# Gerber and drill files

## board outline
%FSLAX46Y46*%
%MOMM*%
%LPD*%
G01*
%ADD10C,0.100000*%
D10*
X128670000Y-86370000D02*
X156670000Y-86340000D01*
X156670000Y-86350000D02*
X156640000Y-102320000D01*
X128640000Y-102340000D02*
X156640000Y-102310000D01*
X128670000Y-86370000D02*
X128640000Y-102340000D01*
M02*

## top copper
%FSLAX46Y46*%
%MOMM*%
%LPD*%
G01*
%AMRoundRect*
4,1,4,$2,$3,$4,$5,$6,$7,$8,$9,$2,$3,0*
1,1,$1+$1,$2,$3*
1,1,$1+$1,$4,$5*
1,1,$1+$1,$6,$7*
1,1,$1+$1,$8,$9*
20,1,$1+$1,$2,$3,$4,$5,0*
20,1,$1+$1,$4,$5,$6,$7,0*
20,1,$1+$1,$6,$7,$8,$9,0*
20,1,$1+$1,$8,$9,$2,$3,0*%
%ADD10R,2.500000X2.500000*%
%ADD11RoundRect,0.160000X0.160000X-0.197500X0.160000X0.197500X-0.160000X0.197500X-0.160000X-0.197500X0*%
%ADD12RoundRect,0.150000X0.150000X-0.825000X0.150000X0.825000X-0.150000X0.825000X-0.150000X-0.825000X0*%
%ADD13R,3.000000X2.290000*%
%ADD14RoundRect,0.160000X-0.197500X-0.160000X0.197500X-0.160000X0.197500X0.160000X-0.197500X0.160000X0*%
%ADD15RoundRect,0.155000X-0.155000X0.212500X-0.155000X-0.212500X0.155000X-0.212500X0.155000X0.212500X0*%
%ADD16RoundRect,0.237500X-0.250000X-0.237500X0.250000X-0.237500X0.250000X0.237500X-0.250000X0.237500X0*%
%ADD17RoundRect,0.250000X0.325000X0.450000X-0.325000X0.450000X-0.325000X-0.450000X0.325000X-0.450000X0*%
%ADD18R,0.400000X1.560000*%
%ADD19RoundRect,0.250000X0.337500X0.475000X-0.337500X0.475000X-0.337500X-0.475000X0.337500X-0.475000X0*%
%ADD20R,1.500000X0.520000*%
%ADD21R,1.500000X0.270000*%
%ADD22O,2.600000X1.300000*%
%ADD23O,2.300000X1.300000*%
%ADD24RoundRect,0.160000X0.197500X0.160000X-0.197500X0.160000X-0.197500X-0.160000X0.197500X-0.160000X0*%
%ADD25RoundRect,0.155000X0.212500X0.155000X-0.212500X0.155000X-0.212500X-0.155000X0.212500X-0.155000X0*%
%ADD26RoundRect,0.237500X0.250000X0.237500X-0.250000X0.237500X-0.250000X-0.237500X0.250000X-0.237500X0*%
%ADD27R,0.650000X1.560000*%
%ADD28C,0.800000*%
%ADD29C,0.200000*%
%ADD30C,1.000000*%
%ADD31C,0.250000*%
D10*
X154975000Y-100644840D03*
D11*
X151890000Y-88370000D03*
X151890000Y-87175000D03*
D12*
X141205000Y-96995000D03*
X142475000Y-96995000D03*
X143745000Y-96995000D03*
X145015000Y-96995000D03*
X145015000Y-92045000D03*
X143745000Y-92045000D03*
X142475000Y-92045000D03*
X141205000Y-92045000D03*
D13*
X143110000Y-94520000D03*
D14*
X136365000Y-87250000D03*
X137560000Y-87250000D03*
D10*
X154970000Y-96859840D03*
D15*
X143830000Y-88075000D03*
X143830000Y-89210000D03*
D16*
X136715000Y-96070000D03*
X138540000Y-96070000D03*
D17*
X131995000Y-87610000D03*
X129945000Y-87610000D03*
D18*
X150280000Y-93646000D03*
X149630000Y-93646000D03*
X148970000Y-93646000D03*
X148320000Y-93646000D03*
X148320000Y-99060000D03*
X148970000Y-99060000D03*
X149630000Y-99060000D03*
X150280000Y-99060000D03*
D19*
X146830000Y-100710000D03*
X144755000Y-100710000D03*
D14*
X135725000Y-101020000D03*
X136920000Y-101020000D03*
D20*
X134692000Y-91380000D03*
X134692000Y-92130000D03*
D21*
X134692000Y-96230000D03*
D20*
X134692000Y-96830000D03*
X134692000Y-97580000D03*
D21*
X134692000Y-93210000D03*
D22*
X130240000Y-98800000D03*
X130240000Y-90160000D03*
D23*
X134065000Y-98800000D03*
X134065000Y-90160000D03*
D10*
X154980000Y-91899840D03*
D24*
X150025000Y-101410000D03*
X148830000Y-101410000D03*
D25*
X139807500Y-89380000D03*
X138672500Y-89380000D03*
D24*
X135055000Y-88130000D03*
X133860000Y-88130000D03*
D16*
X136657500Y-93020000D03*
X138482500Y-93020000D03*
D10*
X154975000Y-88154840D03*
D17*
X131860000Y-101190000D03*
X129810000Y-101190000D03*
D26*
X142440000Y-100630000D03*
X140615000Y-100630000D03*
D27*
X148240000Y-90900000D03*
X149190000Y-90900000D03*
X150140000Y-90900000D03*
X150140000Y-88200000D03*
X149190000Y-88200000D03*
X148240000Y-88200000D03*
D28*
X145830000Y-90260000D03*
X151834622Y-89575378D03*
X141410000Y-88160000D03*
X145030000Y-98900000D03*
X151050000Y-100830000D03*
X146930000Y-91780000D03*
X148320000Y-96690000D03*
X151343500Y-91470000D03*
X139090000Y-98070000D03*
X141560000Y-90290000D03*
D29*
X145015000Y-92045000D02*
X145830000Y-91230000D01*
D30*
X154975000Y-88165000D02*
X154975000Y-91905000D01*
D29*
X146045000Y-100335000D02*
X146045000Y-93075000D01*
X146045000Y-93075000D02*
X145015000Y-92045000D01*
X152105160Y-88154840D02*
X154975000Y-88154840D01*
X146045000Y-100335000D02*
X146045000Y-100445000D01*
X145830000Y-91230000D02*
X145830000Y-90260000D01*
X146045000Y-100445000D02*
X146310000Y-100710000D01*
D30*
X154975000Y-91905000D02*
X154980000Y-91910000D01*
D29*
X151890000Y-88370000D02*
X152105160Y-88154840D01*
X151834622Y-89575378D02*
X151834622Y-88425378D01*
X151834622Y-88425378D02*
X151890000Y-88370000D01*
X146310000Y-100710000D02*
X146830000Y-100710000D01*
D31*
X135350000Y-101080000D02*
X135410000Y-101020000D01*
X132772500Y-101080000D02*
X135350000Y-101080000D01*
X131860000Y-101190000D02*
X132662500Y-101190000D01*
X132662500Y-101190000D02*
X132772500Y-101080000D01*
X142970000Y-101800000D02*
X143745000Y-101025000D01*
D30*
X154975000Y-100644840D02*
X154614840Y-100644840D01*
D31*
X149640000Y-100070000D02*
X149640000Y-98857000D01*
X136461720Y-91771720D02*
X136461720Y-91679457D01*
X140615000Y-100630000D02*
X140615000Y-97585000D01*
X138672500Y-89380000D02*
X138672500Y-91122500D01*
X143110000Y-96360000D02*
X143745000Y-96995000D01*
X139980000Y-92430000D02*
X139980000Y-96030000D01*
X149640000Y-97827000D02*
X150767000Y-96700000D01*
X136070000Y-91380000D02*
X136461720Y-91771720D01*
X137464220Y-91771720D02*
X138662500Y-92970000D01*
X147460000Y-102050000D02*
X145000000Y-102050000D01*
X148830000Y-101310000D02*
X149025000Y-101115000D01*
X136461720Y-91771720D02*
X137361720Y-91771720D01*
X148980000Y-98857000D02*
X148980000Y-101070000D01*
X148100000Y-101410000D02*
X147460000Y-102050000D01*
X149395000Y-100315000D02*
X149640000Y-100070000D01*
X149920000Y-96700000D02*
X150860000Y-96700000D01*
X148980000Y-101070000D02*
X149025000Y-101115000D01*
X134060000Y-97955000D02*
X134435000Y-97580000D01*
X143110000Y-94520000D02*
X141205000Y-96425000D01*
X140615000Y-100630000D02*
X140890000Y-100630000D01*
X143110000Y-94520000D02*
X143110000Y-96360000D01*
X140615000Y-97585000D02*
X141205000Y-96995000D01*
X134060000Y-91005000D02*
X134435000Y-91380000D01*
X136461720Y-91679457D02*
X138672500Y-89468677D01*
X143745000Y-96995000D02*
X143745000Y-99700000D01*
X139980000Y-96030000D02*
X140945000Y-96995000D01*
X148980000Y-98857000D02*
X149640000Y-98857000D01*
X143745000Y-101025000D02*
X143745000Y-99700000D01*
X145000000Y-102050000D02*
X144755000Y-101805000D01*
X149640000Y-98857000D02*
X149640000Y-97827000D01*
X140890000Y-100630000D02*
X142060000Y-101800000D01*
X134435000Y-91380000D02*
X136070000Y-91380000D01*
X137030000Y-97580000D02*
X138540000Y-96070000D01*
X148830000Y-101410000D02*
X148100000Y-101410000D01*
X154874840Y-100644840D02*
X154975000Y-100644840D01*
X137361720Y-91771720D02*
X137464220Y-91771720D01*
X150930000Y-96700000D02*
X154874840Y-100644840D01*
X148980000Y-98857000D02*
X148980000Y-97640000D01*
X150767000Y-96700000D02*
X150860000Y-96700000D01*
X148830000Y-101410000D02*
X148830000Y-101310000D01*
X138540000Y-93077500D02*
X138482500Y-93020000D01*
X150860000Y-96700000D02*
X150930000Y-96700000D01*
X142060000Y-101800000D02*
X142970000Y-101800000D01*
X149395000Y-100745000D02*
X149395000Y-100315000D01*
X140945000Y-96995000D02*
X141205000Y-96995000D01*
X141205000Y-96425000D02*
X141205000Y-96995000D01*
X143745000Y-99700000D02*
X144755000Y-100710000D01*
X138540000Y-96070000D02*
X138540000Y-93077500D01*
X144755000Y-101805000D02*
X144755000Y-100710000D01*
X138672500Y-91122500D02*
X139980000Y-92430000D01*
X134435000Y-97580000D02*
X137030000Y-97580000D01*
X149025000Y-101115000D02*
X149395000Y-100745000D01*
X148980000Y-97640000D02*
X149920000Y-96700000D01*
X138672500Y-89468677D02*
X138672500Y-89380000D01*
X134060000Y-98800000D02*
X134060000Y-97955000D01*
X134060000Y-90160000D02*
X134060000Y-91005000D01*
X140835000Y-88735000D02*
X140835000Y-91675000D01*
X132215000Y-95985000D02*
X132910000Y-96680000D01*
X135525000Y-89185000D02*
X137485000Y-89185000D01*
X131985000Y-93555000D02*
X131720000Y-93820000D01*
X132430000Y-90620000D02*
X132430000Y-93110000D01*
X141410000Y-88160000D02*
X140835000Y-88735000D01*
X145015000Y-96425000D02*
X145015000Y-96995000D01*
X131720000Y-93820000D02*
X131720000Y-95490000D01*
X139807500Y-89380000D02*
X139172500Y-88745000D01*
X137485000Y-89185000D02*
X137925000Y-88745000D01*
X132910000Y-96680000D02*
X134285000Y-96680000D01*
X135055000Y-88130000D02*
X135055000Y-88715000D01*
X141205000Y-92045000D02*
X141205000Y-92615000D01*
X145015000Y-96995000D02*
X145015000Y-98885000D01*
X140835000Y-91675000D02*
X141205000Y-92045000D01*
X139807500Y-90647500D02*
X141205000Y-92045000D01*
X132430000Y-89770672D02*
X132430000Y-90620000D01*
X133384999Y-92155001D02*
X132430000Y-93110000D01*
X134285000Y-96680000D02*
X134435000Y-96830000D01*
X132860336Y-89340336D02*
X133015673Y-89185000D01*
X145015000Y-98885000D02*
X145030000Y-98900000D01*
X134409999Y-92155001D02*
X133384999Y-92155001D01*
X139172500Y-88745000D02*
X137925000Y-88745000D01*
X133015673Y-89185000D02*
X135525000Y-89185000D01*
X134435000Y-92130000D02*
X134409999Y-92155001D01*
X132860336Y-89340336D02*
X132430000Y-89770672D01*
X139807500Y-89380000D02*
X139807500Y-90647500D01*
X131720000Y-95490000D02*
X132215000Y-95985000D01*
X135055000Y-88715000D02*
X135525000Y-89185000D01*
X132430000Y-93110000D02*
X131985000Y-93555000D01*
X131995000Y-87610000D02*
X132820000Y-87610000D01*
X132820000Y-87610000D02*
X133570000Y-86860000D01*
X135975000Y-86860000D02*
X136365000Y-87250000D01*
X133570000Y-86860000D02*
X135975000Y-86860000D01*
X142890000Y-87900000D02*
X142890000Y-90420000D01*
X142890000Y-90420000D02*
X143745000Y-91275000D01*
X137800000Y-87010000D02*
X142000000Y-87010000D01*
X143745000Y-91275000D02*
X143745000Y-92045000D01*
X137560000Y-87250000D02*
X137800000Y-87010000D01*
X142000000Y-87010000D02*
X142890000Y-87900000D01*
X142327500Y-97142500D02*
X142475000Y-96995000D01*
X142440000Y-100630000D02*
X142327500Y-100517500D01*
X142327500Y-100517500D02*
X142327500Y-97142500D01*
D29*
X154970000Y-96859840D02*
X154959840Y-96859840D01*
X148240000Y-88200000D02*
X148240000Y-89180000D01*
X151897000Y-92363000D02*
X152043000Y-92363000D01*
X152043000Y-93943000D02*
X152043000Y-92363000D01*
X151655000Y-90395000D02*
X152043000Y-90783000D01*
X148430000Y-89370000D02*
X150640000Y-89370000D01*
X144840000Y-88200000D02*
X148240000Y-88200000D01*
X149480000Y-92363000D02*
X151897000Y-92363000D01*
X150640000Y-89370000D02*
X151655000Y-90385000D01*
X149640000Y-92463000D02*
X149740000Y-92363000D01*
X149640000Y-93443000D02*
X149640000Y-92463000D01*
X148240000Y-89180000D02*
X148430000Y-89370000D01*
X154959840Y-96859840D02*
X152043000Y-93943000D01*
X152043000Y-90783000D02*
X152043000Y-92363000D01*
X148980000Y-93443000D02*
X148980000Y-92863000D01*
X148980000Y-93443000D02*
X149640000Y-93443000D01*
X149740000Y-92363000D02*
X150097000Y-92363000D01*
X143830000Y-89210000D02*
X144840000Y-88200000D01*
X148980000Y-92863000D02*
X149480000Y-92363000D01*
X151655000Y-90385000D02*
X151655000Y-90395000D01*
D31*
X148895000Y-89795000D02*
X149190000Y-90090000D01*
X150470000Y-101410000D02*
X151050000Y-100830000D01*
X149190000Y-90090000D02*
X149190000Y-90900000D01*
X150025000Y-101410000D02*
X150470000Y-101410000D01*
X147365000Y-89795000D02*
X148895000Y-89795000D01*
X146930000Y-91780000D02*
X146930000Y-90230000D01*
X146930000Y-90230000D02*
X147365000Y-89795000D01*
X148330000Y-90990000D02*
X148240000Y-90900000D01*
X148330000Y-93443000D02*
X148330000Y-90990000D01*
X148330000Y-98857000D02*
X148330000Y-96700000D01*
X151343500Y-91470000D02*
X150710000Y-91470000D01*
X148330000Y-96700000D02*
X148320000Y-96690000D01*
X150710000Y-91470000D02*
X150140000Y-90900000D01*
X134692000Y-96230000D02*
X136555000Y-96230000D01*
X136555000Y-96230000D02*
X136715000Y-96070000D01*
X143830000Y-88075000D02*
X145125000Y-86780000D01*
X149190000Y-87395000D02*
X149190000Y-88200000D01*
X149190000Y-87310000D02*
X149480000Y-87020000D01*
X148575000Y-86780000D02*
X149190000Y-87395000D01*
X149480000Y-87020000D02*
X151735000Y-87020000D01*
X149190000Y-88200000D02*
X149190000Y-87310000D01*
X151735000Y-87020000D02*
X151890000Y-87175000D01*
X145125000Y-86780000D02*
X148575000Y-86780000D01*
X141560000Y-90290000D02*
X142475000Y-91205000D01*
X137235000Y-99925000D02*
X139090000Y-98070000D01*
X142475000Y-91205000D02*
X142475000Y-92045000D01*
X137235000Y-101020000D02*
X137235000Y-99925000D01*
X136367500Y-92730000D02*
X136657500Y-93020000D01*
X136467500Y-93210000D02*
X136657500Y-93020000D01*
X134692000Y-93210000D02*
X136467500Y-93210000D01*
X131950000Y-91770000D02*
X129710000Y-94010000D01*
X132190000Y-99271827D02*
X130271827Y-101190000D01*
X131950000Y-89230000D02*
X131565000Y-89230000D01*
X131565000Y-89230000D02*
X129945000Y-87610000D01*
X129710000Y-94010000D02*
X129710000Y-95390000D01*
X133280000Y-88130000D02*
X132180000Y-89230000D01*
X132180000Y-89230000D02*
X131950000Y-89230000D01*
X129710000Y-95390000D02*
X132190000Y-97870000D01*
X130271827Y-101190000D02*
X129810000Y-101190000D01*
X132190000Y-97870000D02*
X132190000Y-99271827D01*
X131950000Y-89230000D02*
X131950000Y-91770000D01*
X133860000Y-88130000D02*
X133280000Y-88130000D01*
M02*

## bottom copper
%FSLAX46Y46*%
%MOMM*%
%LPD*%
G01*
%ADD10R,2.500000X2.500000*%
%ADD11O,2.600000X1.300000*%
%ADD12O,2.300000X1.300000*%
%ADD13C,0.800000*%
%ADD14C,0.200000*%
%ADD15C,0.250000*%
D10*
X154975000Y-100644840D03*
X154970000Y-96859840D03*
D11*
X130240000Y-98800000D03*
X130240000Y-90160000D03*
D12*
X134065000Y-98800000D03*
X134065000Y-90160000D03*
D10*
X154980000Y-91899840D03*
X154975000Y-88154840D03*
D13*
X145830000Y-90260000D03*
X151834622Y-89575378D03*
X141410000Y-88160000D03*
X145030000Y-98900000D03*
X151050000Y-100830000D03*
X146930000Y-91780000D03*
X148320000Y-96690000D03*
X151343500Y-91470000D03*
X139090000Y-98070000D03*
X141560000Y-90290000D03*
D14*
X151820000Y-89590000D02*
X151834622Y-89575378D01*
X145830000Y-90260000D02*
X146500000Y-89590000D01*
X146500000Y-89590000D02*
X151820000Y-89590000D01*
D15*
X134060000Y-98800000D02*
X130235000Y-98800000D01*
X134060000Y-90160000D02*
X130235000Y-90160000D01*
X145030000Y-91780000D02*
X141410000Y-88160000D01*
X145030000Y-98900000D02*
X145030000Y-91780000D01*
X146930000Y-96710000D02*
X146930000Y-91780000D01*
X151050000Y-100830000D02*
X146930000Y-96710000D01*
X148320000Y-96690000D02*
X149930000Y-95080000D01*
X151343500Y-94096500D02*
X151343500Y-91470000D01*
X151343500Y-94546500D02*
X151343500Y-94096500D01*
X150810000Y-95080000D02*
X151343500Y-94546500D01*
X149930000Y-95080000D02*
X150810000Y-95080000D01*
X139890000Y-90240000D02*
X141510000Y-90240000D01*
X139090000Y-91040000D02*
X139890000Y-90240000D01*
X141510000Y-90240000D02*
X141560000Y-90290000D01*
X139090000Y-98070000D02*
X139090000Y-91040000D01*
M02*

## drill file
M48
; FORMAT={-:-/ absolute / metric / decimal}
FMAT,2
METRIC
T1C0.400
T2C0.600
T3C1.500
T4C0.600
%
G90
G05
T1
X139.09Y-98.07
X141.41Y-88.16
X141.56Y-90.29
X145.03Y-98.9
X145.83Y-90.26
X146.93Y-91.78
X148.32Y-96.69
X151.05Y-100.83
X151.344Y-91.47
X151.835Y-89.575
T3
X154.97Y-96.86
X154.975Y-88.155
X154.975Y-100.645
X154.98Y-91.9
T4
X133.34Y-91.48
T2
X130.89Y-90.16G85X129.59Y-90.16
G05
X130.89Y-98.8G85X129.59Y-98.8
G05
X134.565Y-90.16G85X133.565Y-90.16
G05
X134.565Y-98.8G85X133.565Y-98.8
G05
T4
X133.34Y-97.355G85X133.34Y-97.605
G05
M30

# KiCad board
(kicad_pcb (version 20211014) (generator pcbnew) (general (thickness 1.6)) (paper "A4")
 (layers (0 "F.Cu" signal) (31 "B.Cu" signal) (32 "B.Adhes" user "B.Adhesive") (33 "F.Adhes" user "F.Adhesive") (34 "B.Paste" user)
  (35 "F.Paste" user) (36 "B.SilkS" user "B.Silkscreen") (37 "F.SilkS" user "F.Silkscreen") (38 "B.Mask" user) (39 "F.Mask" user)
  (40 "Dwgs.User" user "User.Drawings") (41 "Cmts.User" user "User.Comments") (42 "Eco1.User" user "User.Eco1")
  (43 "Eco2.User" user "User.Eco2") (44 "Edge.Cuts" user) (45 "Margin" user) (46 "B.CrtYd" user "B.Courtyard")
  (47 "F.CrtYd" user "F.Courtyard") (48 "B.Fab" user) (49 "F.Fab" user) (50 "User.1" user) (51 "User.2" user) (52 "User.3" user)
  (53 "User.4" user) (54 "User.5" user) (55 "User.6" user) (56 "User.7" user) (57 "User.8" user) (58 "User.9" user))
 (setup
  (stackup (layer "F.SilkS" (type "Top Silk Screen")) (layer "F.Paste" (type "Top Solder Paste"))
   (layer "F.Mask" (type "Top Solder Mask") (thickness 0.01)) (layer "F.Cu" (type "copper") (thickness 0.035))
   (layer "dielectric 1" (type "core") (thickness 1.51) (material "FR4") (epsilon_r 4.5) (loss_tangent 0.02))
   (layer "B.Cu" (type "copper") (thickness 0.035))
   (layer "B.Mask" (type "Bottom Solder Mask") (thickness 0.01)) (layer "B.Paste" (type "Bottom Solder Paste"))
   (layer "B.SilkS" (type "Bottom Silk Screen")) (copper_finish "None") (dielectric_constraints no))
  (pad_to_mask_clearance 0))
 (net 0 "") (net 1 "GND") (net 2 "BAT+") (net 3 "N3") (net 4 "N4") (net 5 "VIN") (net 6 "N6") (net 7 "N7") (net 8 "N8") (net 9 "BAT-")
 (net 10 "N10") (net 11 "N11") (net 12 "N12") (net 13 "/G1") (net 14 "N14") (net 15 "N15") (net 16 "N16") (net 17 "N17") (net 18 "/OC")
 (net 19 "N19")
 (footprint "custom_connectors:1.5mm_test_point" (layer "F.Cu") (at 154.975 100.655)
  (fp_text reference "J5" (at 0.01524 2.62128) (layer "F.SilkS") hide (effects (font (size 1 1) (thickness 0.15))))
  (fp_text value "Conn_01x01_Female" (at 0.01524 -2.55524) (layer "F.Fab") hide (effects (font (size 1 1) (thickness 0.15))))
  (pad "1" thru_hole rect (at 0 -0.01016) (size 2.5 2.5) (drill 1.5) (layers *.Cu *.Mask) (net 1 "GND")))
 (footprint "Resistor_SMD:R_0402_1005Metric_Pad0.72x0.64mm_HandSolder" (layer "F.Cu") (at 151.89 87.7725 90)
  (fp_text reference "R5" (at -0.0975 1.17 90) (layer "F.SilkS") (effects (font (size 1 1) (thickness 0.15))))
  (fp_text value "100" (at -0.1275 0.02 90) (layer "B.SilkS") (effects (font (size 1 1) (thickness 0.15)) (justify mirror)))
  (pad "1" smd roundrect (at -0.5975 0 90) (size 0.715 0.64) (layers "F.Cu" "F.Paste" "F.Mask") (roundrect_rratio 0.25) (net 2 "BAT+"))
  (pad "2" smd roundrect (at 0.5975 0 90) (size 0.715 0.64) (layers "F.Cu" "F.Paste" "F.Mask") (roundrect_rratio 0.25) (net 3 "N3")))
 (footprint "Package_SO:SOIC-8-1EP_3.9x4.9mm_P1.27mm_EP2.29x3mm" (layer "F.Cu") (at 143.11 94.52 90)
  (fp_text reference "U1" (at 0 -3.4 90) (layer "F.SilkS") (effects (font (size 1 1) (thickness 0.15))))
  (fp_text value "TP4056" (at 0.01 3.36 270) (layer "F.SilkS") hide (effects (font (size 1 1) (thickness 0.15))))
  (pad "" smd roundrect (at 0.57 0.75 90) (size 0.92 1.21) (layers "F.Paste") (roundrect_rratio 0.25))
  (pad "" smd roundrect (at 0.57 -0.75 90) (size 0.92 1.21) (layers "F.Paste") (roundrect_rratio 0.25))
  (pad "" smd roundrect (at -0.57 0.75 90) (size 0.92 1.21) (layers "F.Paste") (roundrect_rratio 0.25))
  (pad "" smd roundrect (at -0.57 -0.75 90) (size 0.92 1.21) (layers "F.Paste") (roundrect_rratio 0.25))
  (pad "1" smd roundrect (at -2.475 -1.905 90) (size 1.95 0.6) (layers "F.Cu" "F.Paste" "F.Mask") (roundrect_rratio 0.25) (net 1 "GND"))
  (pad "2" smd roundrect (at -2.475 -0.635 90) (size 1.95 0.6) (layers "F.Cu" "F.Paste" "F.Mask") (roundrect_rratio 0.25) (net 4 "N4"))
  (pad "3" smd roundrect (at -2.475 0.635 90) (size 1.95 0.6) (layers "F.Cu" "F.Paste" "F.Mask") (roundrect_rratio 0.25) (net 1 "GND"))
  (pad "4" smd roundrect (at -2.475 1.905 90) (size 1.95 0.6) (layers "F.Cu" "F.Paste" "F.Mask") (roundrect_rratio 0.25) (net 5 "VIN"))
  (pad "5" smd roundrect (at 2.475 1.905 90) (size 1.95 0.6) (layers "F.Cu" "F.Paste" "F.Mask") (roundrect_rratio 0.25) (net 2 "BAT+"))
  (pad "6" smd roundrect (at 2.475 0.635 90) (size 1.95 0.6) (layers "F.Cu" "F.Paste" "F.Mask") (roundrect_rratio 0.25) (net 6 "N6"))
  (pad "7" smd roundrect (at 2.475 -0.635 90) (size 1.95 0.6) (layers "F.Cu" "F.Paste" "F.Mask") (roundrect_rratio 0.25) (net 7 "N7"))
  (pad "8" smd roundrect (at 2.475 -1.905 90) (size 1.95 0.6) (layers "F.Cu" "F.Paste" "F.Mask") (roundrect_rratio 0.25) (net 5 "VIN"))
  (pad "9" smd rect (at 0 0 90) (size 2.29 3) (layers "F.Cu" "F.Mask") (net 1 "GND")))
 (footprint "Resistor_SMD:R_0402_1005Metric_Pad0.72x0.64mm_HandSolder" (layer "F.Cu") (at 136.9625 87.25)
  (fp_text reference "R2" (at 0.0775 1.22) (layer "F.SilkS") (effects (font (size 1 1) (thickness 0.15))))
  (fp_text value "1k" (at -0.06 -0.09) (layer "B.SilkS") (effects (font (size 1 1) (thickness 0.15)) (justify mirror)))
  (pad "1" smd roundrect (at -0.5975 0) (size 0.715 0.64) (layers "F.Cu" "F.Paste" "F.Mask") (roundrect_rratio 0.25) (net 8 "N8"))
  (pad "2" smd roundrect (at 0.5975 0) (size 0.715 0.64) (layers "F.Cu" "F.Paste" "F.Mask") (roundrect_rratio 0.25) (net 6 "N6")))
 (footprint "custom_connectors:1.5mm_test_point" (layer "F.Cu") (at 154.97 96.87)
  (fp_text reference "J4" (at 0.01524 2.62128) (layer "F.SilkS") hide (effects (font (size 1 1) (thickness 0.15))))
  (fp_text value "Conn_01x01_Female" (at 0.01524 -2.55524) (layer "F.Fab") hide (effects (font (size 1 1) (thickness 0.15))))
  (pad "1" thru_hole rect (at 0 -0.01016) (size 2.5 2.5) (drill 1.5) (layers *.Cu *.Mask) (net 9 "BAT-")))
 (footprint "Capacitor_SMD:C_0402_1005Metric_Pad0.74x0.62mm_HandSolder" (layer "F.Cu") (at 143.83 88.6425 -90)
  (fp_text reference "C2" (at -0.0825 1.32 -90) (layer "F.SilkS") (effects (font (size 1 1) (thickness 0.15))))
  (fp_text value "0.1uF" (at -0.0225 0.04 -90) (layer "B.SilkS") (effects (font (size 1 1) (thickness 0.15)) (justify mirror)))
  (pad "1" smd roundrect (at -0.5675 0 270) (size 0.735 0.62) (layers "F.Cu" "F.Paste" "F.Mask") (roundrect_rratio 0.25) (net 3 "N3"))
  (pad "2" smd roundrect (at 0.5675 0 270) (size 0.735 0.62) (layers "F.Cu" "F.Paste" "F.Mask") (roundrect_rratio 0.25) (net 9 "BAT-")))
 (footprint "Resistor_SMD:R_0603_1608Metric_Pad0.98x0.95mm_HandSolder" (layer "F.Cu") (at 137.6275 96.07)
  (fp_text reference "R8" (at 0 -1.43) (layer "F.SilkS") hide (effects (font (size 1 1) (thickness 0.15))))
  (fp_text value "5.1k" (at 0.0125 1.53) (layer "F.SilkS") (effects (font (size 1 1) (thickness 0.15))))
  (pad "1" smd roundrect (at -0.9125 0) (size 0.975 0.95) (layers "F.Cu" "F.Paste" "F.Mask") (roundrect_rratio 0.25) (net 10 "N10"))
  (pad "2" smd roundrect (at 0.9125 0) (size 0.975 0.95) (layers "F.Cu" "F.Paste" "F.Mask") (roundrect_rratio 0.25) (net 1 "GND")))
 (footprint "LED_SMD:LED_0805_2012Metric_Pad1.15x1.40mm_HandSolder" (layer "F.Cu") (at 130.97 87.61 180)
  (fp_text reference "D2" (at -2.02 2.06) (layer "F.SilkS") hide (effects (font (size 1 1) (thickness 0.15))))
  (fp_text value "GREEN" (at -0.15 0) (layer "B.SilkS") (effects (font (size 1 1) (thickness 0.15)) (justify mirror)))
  (pad "1" smd roundrect (at -1.025 0 180) (size 1.15 1.4) (layers "F.Cu" "F.Paste" "F.Mask") (roundrect_rratio 0.2173913043) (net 8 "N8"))
  (pad "2" smd roundrect (at 1.025 0 180) (size 1.15 1.4) (layers "F.Cu" "F.Paste" "F.Mask") (roundrect_rratio 0.2173913043) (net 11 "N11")))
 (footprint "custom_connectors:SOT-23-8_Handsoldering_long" (layer "F.Cu") (at 149.3 94.996 -90)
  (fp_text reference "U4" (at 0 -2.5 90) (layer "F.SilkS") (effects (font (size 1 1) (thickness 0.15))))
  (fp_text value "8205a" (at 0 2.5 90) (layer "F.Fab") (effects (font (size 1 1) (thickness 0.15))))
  (pad "1" smd rect (at -1.35 -0.98 270) (size 1.56 0.4) (layers "F.Cu" "F.Paste" "F.Mask") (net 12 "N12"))
  (pad "2" smd rect (at -1.35 -0.33 270) (size 1.56 0.4) (layers "F.Cu" "F.Paste" "F.Mask") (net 9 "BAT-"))
  (pad "3" smd rect (at -1.35 0.33 270) (size 1.56 0.4) (layers "F.Cu" "F.Paste" "F.Mask") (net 9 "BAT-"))
  (pad "4" smd rect (at -1.35 0.98 270) (size 1.56 0.4) (layers "F.Cu" "F.Paste" "F.Mask") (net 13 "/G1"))
  (pad "5" smd rect (at 4.064 0.98 270) (size 1.56 0.4) (layers "F.Cu" "F.Paste" "F.Mask") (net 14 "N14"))
  (pad "6" smd rect (at 4.064 0.33 270) (size 1.56 0.4) (layers "F.Cu" "F.Paste" "F.Mask") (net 1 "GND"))
  (pad "7" smd rect (at 4.064 -0.33 270) (size 1.56 0.4) (layers "F.Cu" "F.Paste" "F.Mask") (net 1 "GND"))
  (pad "8" smd rect (at 4.064 -0.98 270) (size 1.56 0.4) (layers "F.Cu" "F.Paste" "F.Mask") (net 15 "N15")))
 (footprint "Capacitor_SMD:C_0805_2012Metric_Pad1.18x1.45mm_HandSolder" (layer "F.Cu") (at 145.7925 100.71 180)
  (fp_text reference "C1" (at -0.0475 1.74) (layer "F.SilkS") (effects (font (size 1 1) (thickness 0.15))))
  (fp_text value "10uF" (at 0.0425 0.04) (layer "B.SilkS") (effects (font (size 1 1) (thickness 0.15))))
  (pad "1" smd roundrect (at -1.0375 0 180) (size 1.175 1.45) (layers "F.Cu" "F.Paste" "F.Mask") (roundrect_rratio 0.2127659574)
   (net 2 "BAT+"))
  (pad "2" smd roundrect (at 1.0375 0 180) (size 1.175 1.45) (layers "F.Cu" "F.Paste" "F.Mask") (roundrect_rratio 0.2127659574)
   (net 1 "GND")))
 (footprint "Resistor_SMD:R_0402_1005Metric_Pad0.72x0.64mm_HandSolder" (layer "F.Cu") (at 136.3225 101.02)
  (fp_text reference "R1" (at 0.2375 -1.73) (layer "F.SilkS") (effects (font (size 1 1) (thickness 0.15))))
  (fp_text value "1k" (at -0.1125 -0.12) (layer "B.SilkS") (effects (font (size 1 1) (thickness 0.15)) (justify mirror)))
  (pad "1" smd roundrect (at -0.5975 0) (size 0.715 0.64) (layers "F.Cu" "F.Paste" "F.Mask") (roundrect_rratio 0.25) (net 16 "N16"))
  (pad "2" smd roundrect (at 0.5975 0) (size 0.715 0.64) (layers "F.Cu" "F.Paste" "F.Mask") (roundrect_rratio 0.25) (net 7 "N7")))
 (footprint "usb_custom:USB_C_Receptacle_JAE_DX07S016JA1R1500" (layer "F.Cu") (at 131.39 94.48 -90)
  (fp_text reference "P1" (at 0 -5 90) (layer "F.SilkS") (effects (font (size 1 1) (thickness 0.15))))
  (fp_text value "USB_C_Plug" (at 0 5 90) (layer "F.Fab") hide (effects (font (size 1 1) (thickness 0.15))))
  (pad "" np_thru_hole oval (at 3 -1.95 270) (size 0.85 0.6) (drill oval 0.85 0.6) (layers F&B.Cu *.Mask))
  (pad "" np_thru_hole circle (at -3 -1.95 270) (size 0.6 0.6) (drill 0.6) (layers F&B.Cu *.Mask))
  (pad "A1" smd rect (at -3.1 -3.302 270) (size 0.52 1.5) (layers "F.Cu" "F.Paste" "F.Mask") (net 1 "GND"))
  (pad "A4" smd rect (at -2.35 -3.302 270) (size 0.52 1.5) (layers "F.Cu" "F.Paste" "F.Mask") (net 5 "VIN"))
  (pad "A8" smd rect (at 1.75 -3.302 270) (size 0.27 1.5) (layers "F.Cu" "F.Paste" "F.Mask") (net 10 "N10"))
  (pad "A9" smd rect (at 2.35 -3.302 270) (size 0.52 1.5) (layers "F.Cu" "F.Paste" "F.Mask") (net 5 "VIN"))
  (pad "A12" smd rect (at 3.1 -3.302 270) (size 0.52 1.5) (layers "F.Cu" "F.Paste" "F.Mask") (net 1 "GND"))
  (pad "B8" smd rect (at -1.27 -3.302 270) (size 0.27 1.5) (layers "F.Cu" "F.Paste" "F.Mask") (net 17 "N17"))
  (pad "S1" thru_hole oval (at 4.32 1.15 270) (size 1.3 2.6) (drill oval 0.6 1.9) (layers *.Cu *.Mask) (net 1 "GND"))
  (pad "S1" thru_hole oval (at -4.32 1.15 270) (size 1.3 2.6) (drill oval 0.6 1.9) (layers *.Cu *.Mask) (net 1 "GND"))
  (pad "S1" thru_hole oval (at 4.32 -2.675 270) (size 1.3 2.3) (drill oval 0.6 1.6) (layers *.Cu *.Mask) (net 1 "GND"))
  (pad "S1" thru_hole oval (at -4.32 -2.675 270) (size 1.3 2.3) (drill oval 0.6 1.6) (layers *.Cu *.Mask) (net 1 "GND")))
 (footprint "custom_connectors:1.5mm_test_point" (layer "F.Cu") (at 154.98 91.91)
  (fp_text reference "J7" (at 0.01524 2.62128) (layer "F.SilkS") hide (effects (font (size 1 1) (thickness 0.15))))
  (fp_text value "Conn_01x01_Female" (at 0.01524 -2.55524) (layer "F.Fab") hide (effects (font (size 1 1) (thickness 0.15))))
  (pad "1" thru_hole rect (at 0 -0.01016) (size 2.5 2.5) (drill 1.5) (layers *.Cu *.Mask) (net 2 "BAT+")))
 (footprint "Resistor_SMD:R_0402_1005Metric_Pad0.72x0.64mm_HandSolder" (layer "F.Cu") (at 149.4275 101.41 180)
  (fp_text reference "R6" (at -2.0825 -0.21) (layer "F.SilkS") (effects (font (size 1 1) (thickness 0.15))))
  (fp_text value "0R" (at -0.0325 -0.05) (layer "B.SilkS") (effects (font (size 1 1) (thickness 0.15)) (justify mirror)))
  (pad "1" smd roundrect (at -0.5975 0 180) (size 0.715 0.64) (layers "F.Cu" "F.Paste" "F.Mask") (roundrect_rratio 0.25) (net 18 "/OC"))
  (pad "2" smd roundrect (at 0.5975 0 180) (size 0.715 0.64) (layers "F.Cu" "F.Paste" "F.Mask") (roundrect_rratio 0.25) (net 1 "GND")))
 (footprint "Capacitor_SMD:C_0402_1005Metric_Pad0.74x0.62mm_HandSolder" (layer "F.Cu") (at 139.24 89.38 180)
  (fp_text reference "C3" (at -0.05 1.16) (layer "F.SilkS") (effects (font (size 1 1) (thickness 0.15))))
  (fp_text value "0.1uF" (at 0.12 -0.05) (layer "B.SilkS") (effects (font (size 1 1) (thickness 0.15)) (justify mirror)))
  (pad "1" smd roundrect (at -0.5675 0 180) (size 0.735 0.62) (layers "F.Cu" "F.Paste" "F.Mask") (roundrect_rratio 0.25) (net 5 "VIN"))
  (pad "2" smd roundrect (at 0.5675 0 180) (size 0.735 0.62) (layers "F.Cu" "F.Paste" "F.Mask") (roundrect_rratio 0.25) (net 1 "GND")))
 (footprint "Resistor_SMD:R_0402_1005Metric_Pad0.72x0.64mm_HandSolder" (layer "F.Cu") (at 134.4575 88.13 180)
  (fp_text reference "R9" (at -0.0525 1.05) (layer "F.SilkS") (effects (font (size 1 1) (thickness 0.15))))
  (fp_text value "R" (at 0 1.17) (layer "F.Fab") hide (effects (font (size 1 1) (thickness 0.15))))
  (pad "1" smd roundrect (at -0.5975 0 180) (size 0.715 0.64) (layers "F.Cu" "F.Paste" "F.Mask") (roundrect_rratio 0.25) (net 5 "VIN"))
  (pad "2" smd roundrect (at 0.5975 0 180) (size 0.715 0.64) (layers "F.Cu" "F.Paste" "F.Mask") (roundrect_rratio 0.25) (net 11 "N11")))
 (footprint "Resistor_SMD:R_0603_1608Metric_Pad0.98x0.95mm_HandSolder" (layer "F.Cu") (at 137.57 93.02)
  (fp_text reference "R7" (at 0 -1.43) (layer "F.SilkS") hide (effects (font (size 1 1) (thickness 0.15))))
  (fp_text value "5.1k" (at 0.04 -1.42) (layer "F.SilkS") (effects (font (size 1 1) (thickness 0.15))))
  (pad "1" smd roundrect (at -0.9125 0) (size 0.975 0.95) (layers "F.Cu" "F.Paste" "F.Mask") (roundrect_rratio 0.25) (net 17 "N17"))
  (pad "2" smd roundrect (at 0.9125 0) (size 0.975 0.95) (layers "F.Cu" "F.Paste" "F.Mask") (roundrect_rratio 0.25) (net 1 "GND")))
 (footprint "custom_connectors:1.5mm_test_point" (layer "F.Cu") (at 154.975 88.165)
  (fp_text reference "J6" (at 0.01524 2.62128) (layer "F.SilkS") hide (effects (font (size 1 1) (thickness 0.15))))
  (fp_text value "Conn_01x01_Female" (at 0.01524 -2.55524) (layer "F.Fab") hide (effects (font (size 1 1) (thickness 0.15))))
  (pad "1" thru_hole rect (at 0 -0.01016) (size 2.5 2.5) (drill 1.5) (layers *.Cu *.Mask) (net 2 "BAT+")))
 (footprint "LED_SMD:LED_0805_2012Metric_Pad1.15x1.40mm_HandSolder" (layer "F.Cu") (at 130.835 101.19 180)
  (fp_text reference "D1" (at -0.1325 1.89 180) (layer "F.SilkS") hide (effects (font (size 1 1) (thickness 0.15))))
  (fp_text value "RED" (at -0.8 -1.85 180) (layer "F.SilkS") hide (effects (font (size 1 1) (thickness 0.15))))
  (pad "1" smd roundrect (at -1.025 0 180) (size 1.15 1.4) (layers "F.Cu" "F.Paste" "F.Mask") (roundrect_rratio 0.2173913043) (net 16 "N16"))
  (pad "2" smd roundrect (at 1.025 0 180) (size 1.15 1.4) (layers "F.Cu" "F.Paste" "F.Mask") (roundrect_rratio 0.2173913043) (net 11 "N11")))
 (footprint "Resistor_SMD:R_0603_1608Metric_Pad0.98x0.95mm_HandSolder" (layer "F.Cu") (at 141.5275 100.63 180)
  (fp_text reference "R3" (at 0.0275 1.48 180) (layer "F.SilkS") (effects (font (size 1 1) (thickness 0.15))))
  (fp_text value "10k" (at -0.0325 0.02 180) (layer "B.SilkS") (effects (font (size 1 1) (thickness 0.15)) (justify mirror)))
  (pad "1" smd roundrect (at -0.9125 0 180) (size 0.975 0.95) (layers "F.Cu" "F.Paste" "F.Mask") (roundrect_rratio 0.25) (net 4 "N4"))
  (pad "2" smd roundrect (at 0.9125 0 180) (size 0.975 0.95) (layers "F.Cu" "F.Paste" "F.Mask") (roundrect_rratio 0.25) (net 1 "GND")))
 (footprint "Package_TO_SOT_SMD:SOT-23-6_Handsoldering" (layer "F.Cu") (at 149.19 89.55 90)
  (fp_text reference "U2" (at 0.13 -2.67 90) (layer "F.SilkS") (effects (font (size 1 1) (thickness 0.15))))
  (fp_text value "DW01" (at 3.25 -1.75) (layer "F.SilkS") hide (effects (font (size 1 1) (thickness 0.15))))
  (pad "1" smd rect (at -1.35 -0.95 90) (size 1.56 0.65) (layers "F.Cu" "F.Paste" "F.Mask") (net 13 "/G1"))
  (pad "2" smd rect (at -1.35 0 90) (size 1.56 0.65) (layers "F.Cu" "F.Paste" "F.Mask") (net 18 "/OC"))
  (pad "3" smd rect (at -1.35 0.95 90) (size 1.56 0.65) (layers "F.Cu" "F.Paste" "F.Mask") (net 14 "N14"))
  (pad "4" smd rect (at 1.35 0.95 90) (size 1.56 0.65) (layers "F.Cu" "F.Paste" "F.Mask") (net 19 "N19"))
  (pad "5" smd rect (at 1.35 0 90) (size 1.56 0.65) (layers "F.Cu" "F.Paste" "F.Mask") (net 3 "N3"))
  (pad "6" smd rect (at 1.35 -0.95 90) (size 1.56 0.65) (layers "F.Cu" "F.Paste" "F.Mask") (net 9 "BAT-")))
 (gr_line (start 128.67 86.37) (end 156.67 86.34) (layer "Edge.Cuts") (width 0.1))
 (gr_line (start 156.67 86.35) (end 156.64 102.32) (layer "Edge.Cuts") (width 0.1))
 (gr_line (start 128.64 102.34) (end 156.64 102.31) (layer "Edge.Cuts") (width 0.1))
 (gr_line (start 128.67 86.37) (end 128.64 102.34) (layer "Edge.Cuts") (width 0.1))
 (segment (start 145.015 92.045) (end 145.83 91.23) (width 0.2) (layer "F.Cu") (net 2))
 (segment (start 154.975 88.165) (end 154.975 91.905) (width 1) (layer "F.Cu") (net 2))
 (segment (start 146.045 100.335) (end 146.045 93.075) (width 0.2) (layer "F.Cu") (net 2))
 (segment (start 146.045 93.075) (end 145.015 92.045) (width 0.2) (layer "F.Cu") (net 2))
 (segment (start 152.10516 88.15484) (end 154.975 88.15484) (width 0.2) (layer "F.Cu") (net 2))
 (segment (start 146.045 100.335) (end 146.045 100.445) (width 0.2) (layer "F.Cu") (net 2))
 (segment (start 145.83 91.23) (end 145.83 90.26) (width 0.2) (layer "F.Cu") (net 2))
 (segment (start 146.045 100.445) (end 146.31 100.71) (width 0.2) (layer "F.Cu") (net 2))
 (segment (start 154.975 91.905) (end 154.98 91.91) (width 1) (layer "F.Cu") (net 2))
 (segment (start 151.89 88.37) (end 152.10516 88.15484) (width 0.2) (layer "F.Cu") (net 2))
 (segment (start 151.834622 89.575378) (end 151.834622 88.425378) (width 0.2) (layer "F.Cu") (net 2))
 (segment (start 151.834622 88.425378) (end 151.89 88.37) (width 0.2) (layer "F.Cu") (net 2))
 (segment (start 146.31 100.71) (end 146.83 100.71) (width 0.2) (layer "F.Cu") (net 2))
 (via (at 145.83 90.26) (size 0.8) (drill 0.4) (layers "F.Cu" "B.Cu") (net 2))
 (via (at 151.834622 89.575378) (size 0.8) (drill 0.4) (layers "F.Cu" "B.Cu") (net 2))
 (segment (start 151.82 89.59) (end 151.834622 89.575378) (width 0.2) (layer "B.Cu") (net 2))
 (segment (start 145.83 90.26) (end 146.5 89.59) (width 0.2) (layer "B.Cu") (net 2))
 (segment (start 146.5 89.59) (end 151.82 89.59) (width 0.2) (layer "B.Cu") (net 2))
 (segment (start 135.35 101.08) (end 135.41 101.02) (width 0.25) (layer "F.Cu") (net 16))
 (segment (start 132.7725 101.08) (end 135.35 101.08) (width 0.25) (layer "F.Cu") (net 16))
 (segment (start 131.86 101.19) (end 132.6625 101.19) (width 0.25) (layer "F.Cu") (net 16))
 (segment (start 132.6625 101.19) (end 132.7725 101.08) (width 0.25) (layer "F.Cu") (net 16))
 (segment (start 142.97 101.8) (end 143.745 101.025) (width 0.25) (layer "F.Cu") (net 1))
 (segment (start 154.975 100.64484) (end 154.61484 100.64484) (width 1) (layer "F.Cu") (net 1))
 (segment (start 149.64 100.07) (end 149.64 98.857) (width 0.25) (layer "F.Cu") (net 1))
 (segment (start 136.46172 91.77172) (end 136.46172 91.679457) (width 0.25) (layer "F.Cu") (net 1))
 (segment (start 140.615 100.63) (end 140.615 97.585) (width 0.25) (layer "F.Cu") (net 1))
 (segment (start 138.6725 89.38) (end 138.6725 91.1225) (width 0.25) (layer "F.Cu") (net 1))
 (segment (start 143.11 96.36) (end 143.745 96.995) (width 0.25) (layer "F.Cu") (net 1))
 (segment (start 139.98 92.43) (end 139.98 96.03) (width 0.25) (layer "F.Cu") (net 1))
 (segment (start 149.64 97.827) (end 150.767 96.7) (width 0.25) (layer "F.Cu") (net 1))
 (segment (start 136.07 91.38) (end 136.46172 91.77172) (width 0.25) (layer "F.Cu") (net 1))
 (segment (start 137.46422 91.77172) (end 138.6625 92.97) (width 0.25) (layer "F.Cu") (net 1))
 (segment (start 147.46 102.05) (end 145 102.05) (width 0.25) (layer "F.Cu") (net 1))
 (segment (start 148.83 101.31) (end 149.025 101.115) (width 0.25) (layer "F.Cu") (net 1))
 (segment (start 136.46172 91.77172) (end 137.36172 91.77172) (width 0.25) (layer "F.Cu") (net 1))
 (segment (start 148.98 98.857) (end 148.98 101.07) (width 0.25) (layer "F.Cu") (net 1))
 (segment (start 148.1 101.41) (end 147.46 102.05) (width 0.25) (layer "F.Cu") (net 1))
 (segment (start 149.395 100.315) (end 149.64 100.07) (width 0.25) (layer "F.Cu") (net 1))
 (segment (start 149.92 96.7) (end 150.86 96.7) (width 0.25) (layer "F.Cu") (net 1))
 (segment (start 148.98 101.07) (end 149.025 101.115) (width 0.25) (layer "F.Cu") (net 1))
 (segment (start 134.06 97.955) (end 134.435 97.58) (width 0.25) (layer "F.Cu") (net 1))
 (segment (start 143.11 94.52) (end 141.205 96.425) (width 0.25) (layer "F.Cu") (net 1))
 (segment (start 140.615 100.63) (end 140.89 100.63) (width 0.25) (layer "F.Cu") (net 1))
 (segment (start 143.11 94.52) (end 143.11 96.36) (width 0.25) (layer "F.Cu") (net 1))
 (segment (start 140.615 97.585) (end 141.205 96.995) (width 0.25) (layer "F.Cu") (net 1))
 (segment (start 134.06 91.005) (end 134.435 91.38) (width 0.25) (layer "F.Cu") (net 1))
 (segment (start 136.46172 91.679457) (end 138.6725 89.468677) (width 0.25) (layer "F.Cu") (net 1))
 (segment (start 143.745 96.995) (end 143.745 99.7) (width 0.25) (layer "F.Cu") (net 1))
 (segment (start 139.98 96.03) (end 140.945 96.995) (width 0.25) (layer "F.Cu") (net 1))
 (segment (start 148.98 98.857) (end 149.64 98.857) (width 0.25) (layer "F.Cu") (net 1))
 (segment (start 143.745 101.025) (end 143.745 99.7) (width 0.25) (layer "F.Cu") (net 1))
 (segment (start 145 102.05) (end 144.755 101.805) (width 0.25) (layer "F.Cu") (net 1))
 (segment (start 149.64 98.857) (end 149.64 97.827) (width 0.25) (layer "F.Cu") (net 1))
 (segment (start 140.89 100.63) (end 142.06 101.8) (width 0.25) (layer "F.Cu") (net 1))
 (segment (start 134.435 91.38) (end 136.07 91.38) (width 0.25) (layer "F.Cu") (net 1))
 (segment (start 137.03 97.58) (end 138.54 96.07) (width 0.25) (layer "F.Cu") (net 1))
 (segment (start 148.83 101.41) (end 148.1 101.41) (width 0.25) (layer "F.Cu") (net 1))
 (segment (start 154.87484 100.64484) (end 154.975 100.64484) (width 0.25) (layer "F.Cu") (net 1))
 (segment (start 137.36172 91.77172) (end 137.46422 91.77172) (width 0.25) (layer "F.Cu") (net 1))
 (segment (start 150.93 96.7) (end 154.87484 100.64484) (width 0.25) (layer "F.Cu") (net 1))
 (segment (start 148.98 98.857) (end 148.98 97.64) (width 0.25) (layer "F.Cu") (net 1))
 (segment (start 150.767 96.7) (end 150.86 96.7) (width 0.25) (layer "F.Cu") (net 1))
 (segment (start 148.83 101.41) (end 148.83 101.31) (width 0.25) (layer "F.Cu") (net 1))
 (segment (start 138.54 93.0775) (end 138.4825 93.02) (width 0.25) (layer "F.Cu") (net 1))
 (segment (start 150.86 96.7) (end 150.93 96.7) (width 0.25) (layer "F.Cu") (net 1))
 (segment (start 142.06 101.8) (end 142.97 101.8) (width 0.25) (layer "F.Cu") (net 1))
 (segment (start 149.395 100.745) (end 149.395 100.315) (width 0.25) (layer "F.Cu") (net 1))
 (segment (start 140.945 96.995) (end 141.205 96.995) (width 0.25) (layer "F.Cu") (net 1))
 (segment (start 141.205 96.425) (end 141.205 96.995) (width 0.25) (layer "F.Cu") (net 1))
 (segment (start 143.745 99.7) (end 144.755 100.71) (width 0.25) (layer "F.Cu") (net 1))
 (segment (start 138.54 96.07) (end 138.54 93.0775) (width 0.25) (layer "F.Cu") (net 1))
 (segment (start 144.755 101.805) (end 144.755 100.71) (width 0.25) (layer "F.Cu") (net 1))
 (segment (start 138.6725 91.1225) (end 139.98 92.43) (width 0.25) (layer "F.Cu") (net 1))
 (segment (start 134.435 97.58) (end 137.03 97.58) (width 0.25) (layer "F.Cu") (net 1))
 (segment (start 149.025 101.115) (end 149.395 100.745) (width 0.25) (layer "F.Cu") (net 1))
 (segment (start 148.98 97.64) (end 149.92 96.7) (width 0.25) (layer "F.Cu") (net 1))
 (segment (start 138.6725 89.468677) (end 138.6725 89.38) (width 0.25) (layer "F.Cu") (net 1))
 (segment (start 134.06 98.8) (end 134.06 97.955) (width 0.25) (layer "F.Cu") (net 1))
 (segment (start 134.06 90.16) (end 134.06 91.005) (width 0.25) (layer "F.Cu") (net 1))
 (segment (start 134.06 98.8) (end 130.235 98.8) (width 0.25) (layer "B.Cu") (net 1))
 (segment (start 134.06 90.16) (end 130.235 90.16) (width 0.25) (layer "B.Cu") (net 1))
 (segment (start 140.835 88.735) (end 140.835 91.675) (width 0.25) (layer "F.Cu") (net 5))
 (segment (start 132.215 95.985) (end 132.91 96.68) (width 0.25) (layer "F.Cu") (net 5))
 (segment (start 135.525 89.185) (end 137.485 89.185) (width 0.25) (layer "F.Cu") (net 5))
 (segment (start 131.985 93.555) (end 131.72 93.82) (width 0.25) (layer "F.Cu") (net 5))
 (segment (start 132.43 90.62) (end 132.43 93.11) (width 0.25) (layer "F.Cu") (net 5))
 (segment (start 141.41 88.16) (end 140.835 88.735) (width 0.25) (layer "F.Cu") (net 5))
 (segment (start 145.015 96.425) (end 145.015 96.995) (width 0.25) (layer "F.Cu") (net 5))
 (segment (start 131.72 93.82) (end 131.72 95.49) (width 0.25) (layer "F.Cu") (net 5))
 (segment (start 139.8075 89.38) (end 139.1725 88.745) (width 0.25) (layer "F.Cu") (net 5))
 (segment (start 137.485 89.185) (end 137.925 88.745) (width 0.25) (layer "F.Cu") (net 5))
 (segment (start 132.91 96.68) (end 134.285 96.68) (width 0.25) (layer "F.Cu") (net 5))
 (segment (start 135.055 88.13) (end 135.055 88.715) (width 0.25) (layer "F.Cu") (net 5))
 (segment (start 141.205 92.045) (end 141.205 92.615) (width 0.25) (layer "F.Cu") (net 5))
 (segment (start 145.015 96.995) (end 145.015 98.885) (width 0.25) (layer "F.Cu") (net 5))
 (segment (start 140.835 91.675) (end 141.205 92.045) (width 0.25) (layer "F.Cu") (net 5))
 (segment (start 139.8075 90.6475) (end 141.205 92.045) (width 0.25) (layer "F.Cu") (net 5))
 (segment (start 132.43 89.770672) (end 132.43 90.62) (width 0.25) (layer "F.Cu") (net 5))
 (segment (start 133.384999 92.155001) (end 132.43 93.11) (width 0.25) (layer "F.Cu") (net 5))
 (segment (start 134.285 96.68) (end 134.435 96.83) (width 0.25) (layer "F.Cu") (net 5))
 (segment (start 132.860336 89.340336) (end 133.015673 89.185) (width 0.25) (layer "F.Cu") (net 5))
 (segment (start 145.015 98.885) (end 145.03 98.9) (width 0.25) (layer "F.Cu") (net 5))
 (segment (start 134.409999 92.155001) (end 133.384999 92.155001) (width 0.25) (layer "F.Cu") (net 5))
 (segment (start 139.1725 88.745) (end 137.925 88.745) (width 0.25) (layer "F.Cu") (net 5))
 (segment (start 133.015673 89.185) (end 135.525 89.185) (width 0.25) (layer "F.Cu") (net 5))
 (segment (start 134.435 92.13) (end 134.409999 92.155001) (width 0.25) (layer "F.Cu") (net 5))
 (segment (start 132.860336 89.340336) (end 132.43 89.770672) (width 0.25) (layer "F.Cu") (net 5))
 (segment (start 139.8075 89.38) (end 139.8075 90.6475) (width 0.25) (layer "F.Cu") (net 5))
 (segment (start 131.72 95.49) (end 132.215 95.985) (width 0.25) (layer "F.Cu") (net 5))
 (segment (start 135.055 88.715) (end 135.525 89.185) (width 0.25) (layer "F.Cu") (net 5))
 (segment (start 132.43 93.11) (end 131.985 93.555) (width 0.25) (layer "F.Cu") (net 5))
 (via (at 141.41 88.16) (size 0.8) (drill 0.4) (layers "F.Cu" "B.Cu") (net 5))
 (via (at 145.03 98.9) (size 0.8) (drill 0.4) (layers "F.Cu" "B.Cu") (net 5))
 (segment (start 145.03 91.78) (end 141.41 88.16) (width 0.25) (layer "B.Cu") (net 5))
 (segment (start 145.03 98.9) (end 145.03 91.78) (width 0.25) (layer "B.Cu") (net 5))
 (segment (start 131.995 87.61) (end 132.82 87.61) (width 0.25) (layer "F.Cu") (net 8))
 (segment (start 132.82 87.61) (end 133.57 86.86) (width 0.25) (layer "F.Cu") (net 8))
 (segment (start 135.975 86.86) (end 136.365 87.25) (width 0.25) (layer "F.Cu") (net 8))
 (segment (start 133.57 86.86) (end 135.975 86.86) (width 0.25) (layer "F.Cu") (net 8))
 (segment (start 142.89 87.9) (end 142.89 90.42) (width 0.25) (layer "F.Cu") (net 6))
 (segment (start 142.89 90.42) (end 143.745 91.275) (width 0.25) (layer "F.Cu") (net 6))
 (segment (start 137.8 87.01) (end 142 87.01) (width 0.25) (layer "F.Cu") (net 6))
 (segment (start 143.745 91.275) (end 143.745 92.045) (width 0.25) (layer "F.Cu") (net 6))
 (segment (start 137.56 87.25) (end 137.8 87.01) (width 0.25) (layer "F.Cu") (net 6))
 (segment (start 142 87.01) (end 142.89 87.9) (width 0.25) (layer "F.Cu") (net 6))
 (segment (start 142.3275 97.1425) (end 142.475 96.995) (width 0.25) (layer "F.Cu") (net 4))
 (segment (start 142.44 100.63) (end 142.3275 100.5175) (width 0.25) (layer "F.Cu") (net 4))
 (segment (start 142.3275 100.5175) (end 142.3275 97.1425) (width 0.25) (layer "F.Cu") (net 4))
 (segment (start 154.97 96.85984) (end 154.95984 96.85984) (width 0.2) (layer "F.Cu") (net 9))
 (segment (start 148.24 88.2) (end 148.24 89.18) (width 0.2) (layer "F.Cu") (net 9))
 (segment (start 151.897 92.363) (end 152.043 92.363) (width 0.2) (layer "F.Cu") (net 9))
 (segment (start 152.043 93.943) (end 152.043 92.363) (width 0.2) (layer "F.Cu") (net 9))
 (segment (start 151.655 90.395) (end 152.043 90.783) (width 0.2) (layer "F.Cu") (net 9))
 (segment (start 148.43 89.37) (end 150.64 89.37) (width 0.2) (layer "F.Cu") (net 9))
 (segment (start 144.84 88.2) (end 148.24 88.2) (width 0.2) (layer "F.Cu") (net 9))
 (segment (start 149.48 92.363) (end 151.897 92.363) (width 0.2) (layer "F.Cu") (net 9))
 (segment (start 150.64 89.37) (end 151.655 90.385) (width 0.2) (layer "F.Cu") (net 9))
 (segment (start 149.64 92.463) (end 149.74 92.363) (width 0.2) (layer "F.Cu") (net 9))
 (segment (start 149.64 93.443) (end 149.64 92.463) (width 0.2) (layer "F.Cu") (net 9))
 (segment (start 148.24 89.18) (end 148.43 89.37) (width 0.2) (layer "F.Cu") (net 9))
 (segment (start 154.95984 96.85984) (end 152.043 93.943) (width 0.2) (layer "F.Cu") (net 9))
 (segment (start 152.043 90.783) (end 152.043 92.363) (width 0.2) (layer "F.Cu") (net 9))
 (segment (start 148.98 93.443) (end 148.98 92.863) (width 0.2) (layer "F.Cu") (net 9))
 (segment (start 148.98 93.443) (end 149.64 93.443) (width 0.2) (layer "F.Cu") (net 9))
 (segment (start 149.74 92.363) (end 150.097 92.363) (width 0.2) (layer "F.Cu") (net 9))
 (segment (start 143.83 89.21) (end 144.84 88.2) (width 0.2) (layer "F.Cu") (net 9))
 (segment (start 148.98 92.863) (end 149.48 92.363) (width 0.2) (layer "F.Cu") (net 9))
 (segment (start 151.655 90.385) (end 151.655 90.395) (width 0.2) (layer "F.Cu") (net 9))
 (segment (start 148.895 89.795) (end 149.19 90.09) (width 0.25) (layer "F.Cu") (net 18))
 (segment (start 150.47 101.41) (end 151.05 100.83) (width 0.25) (layer "F.Cu") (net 18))
 (segment (start 149.19 90.09) (end 149.19 90.9) (width 0.25) (layer "F.Cu") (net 18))
 (segment (start 150.025 101.41) (end 150.47 101.41) (width 0.25) (layer "F.Cu") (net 18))
 (segment (start 147.365 89.795) (end 148.895 89.795) (width 0.25) (layer "F.Cu") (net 18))
 (segment (start 146.93 91.78) (end 146.93 90.23) (width 0.25) (layer "F.Cu") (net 18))
 (segment (start 146.93 90.23) (end 147.365 89.795) (width 0.25) (layer "F.Cu") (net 18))
 (via (at 151.05 100.83) (size 0.8) (drill 0.4) (layers "F.Cu" "B.Cu") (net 18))
 (via (at 146.93 91.78) (size 0.8) (drill 0.4) (layers "F.Cu" "B.Cu") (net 18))
 (segment (start 146.93 96.71) (end 146.93 91.78) (width 0.25) (layer "B.Cu") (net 18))
 (segment (start 151.05 100.83) (end 146.93 96.71) (width 0.25) (layer "B.Cu") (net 18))
 (segment (start 148.33 90.99) (end 148.24 90.9) (width 0.25) (layer "F.Cu") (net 13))
 (segment (start 148.33 93.443) (end 148.33 90.99) (width 0.25) (layer "F.Cu") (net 13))
 (segment (start 148.33 98.857) (end 148.33 96.7) (width 0.25) (layer "F.Cu") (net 14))
 (segment (start 151.3435 91.47) (end 150.71 91.47) (width 0.25) (layer "F.Cu") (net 14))
 (segment (start 148.33 96.7) (end 148.32 96.69) (width 0.25) (layer "F.Cu") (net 14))
 (segment (start 150.71 91.47) (end 150.14 90.9) (width 0.25) (layer "F.Cu") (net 14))
 (via (at 148.32 96.69) (size 0.8) (drill 0.4) (layers "F.Cu" "B.Cu") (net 14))
 (via (at 151.3435 91.47) (size 0.8) (drill 0.4) (layers "F.Cu" "B.Cu") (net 14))
 (segment (start 148.32 96.69) (end 149.93 95.08) (width 0.25) (layer "B.Cu") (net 14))
 (segment (start 151.3435 94.0965) (end 151.3435 91.47) (width 0.25) (layer "B.Cu") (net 14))
 (segment (start 151.3435 94.5465) (end 151.3435 94.0965) (width 0.25) (layer "B.Cu") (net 14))
 (segment (start 150.81 95.08) (end 151.3435 94.5465) (width 0.25) (layer "B.Cu") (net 14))
 (segment (start 149.93 95.08) (end 150.81 95.08) (width 0.25) (layer "B.Cu") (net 14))
 (segment (start 134.692 96.23) (end 136.555 96.23) (width 0.25) (layer "F.Cu") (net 10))
 (segment (start 136.555 96.23) (end 136.715 96.07) (width 0.25) (layer "F.Cu") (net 10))
 (segment (start 143.83 88.075) (end 145.125 86.78) (width 0.25) (layer "F.Cu") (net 3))
 (segment (start 149.19 87.395) (end 149.19 88.2) (width 0.25) (layer "F.Cu") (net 3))
 (segment (start 149.19 87.31) (end 149.48 87.02) (width 0.25) (layer "F.Cu") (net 3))
 (segment (start 148.575 86.78) (end 149.19 87.395) (width 0.25) (layer "F.Cu") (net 3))
 (segment (start 149.48 87.02) (end 151.735 87.02) (width 0.25) (layer "F.Cu") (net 3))
 (segment (start 149.19 88.2) (end 149.19 87.31) (width 0.25) (layer "F.Cu") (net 3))
 (segment (start 151.735 87.02) (end 151.89 87.175) (width 0.25) (layer "F.Cu") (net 3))
 (segment (start 145.125 86.78) (end 148.575 86.78) (width 0.25) (layer "F.Cu") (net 3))
 (segment (start 141.56 90.29) (end 142.475 91.205) (width 0.25) (layer "F.Cu") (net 7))
 (segment (start 137.235 99.925) (end 139.09 98.07) (width 0.25) (layer "F.Cu") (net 7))
 (segment (start 142.475 91.205) (end 142.475 92.045) (width 0.25) (layer "F.Cu") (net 7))
 (segment (start 137.235 101.02) (end 137.235 99.925) (width 0.25) (layer "F.Cu") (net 7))
 (via (at 139.09 98.07) (size 0.8) (drill 0.4) (layers "F.Cu" "B.Cu") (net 7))
 (via (at 141.56 90.29) (size 0.8) (drill 0.4) (layers "F.Cu" "B.Cu") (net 7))
 (segment (start 139.89 90.24) (end 141.51 90.24) (width 0.25) (layer "B.Cu") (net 7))
 (segment (start 139.09 91.04) (end 139.89 90.24) (width 0.25) (layer "B.Cu") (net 7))
 (segment (start 141.51 90.24) (end 141.56 90.29) (width 0.25) (layer "B.Cu") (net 7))
 (segment (start 139.09 98.07) (end 139.09 91.04) (width 0.25) (layer "B.Cu") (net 7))
 (segment (start 136.3675 92.73) (end 136.6575 93.02) (width 0.25) (layer "F.Cu") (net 17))
 (segment (start 136.4675 93.21) (end 136.6575 93.02) (width 0.25) (layer "F.Cu") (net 17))
 (segment (start 134.692 93.21) (end 136.4675 93.21) (width 0.25) (layer "F.Cu") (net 17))
 (segment (start 131.95 91.77) (end 129.71 94.01) (width 0.25) (layer "F.Cu") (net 11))
 (segment (start 132.19 99.271827) (end 130.271827 101.19) (width 0.25) (layer "F.Cu") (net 11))
 (segment (start 131.95 89.23) (end 131.565 89.23) (width 0.25) (layer "F.Cu") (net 11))
 (segment (start 131.565 89.23) (end 129.945 87.61) (width 0.25) (layer "F.Cu") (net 11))
 (segment (start 129.71 94.01) (end 129.71 95.39) (width 0.25) (layer "F.Cu") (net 11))
 (segment (start 133.28 88.13) (end 132.18 89.23) (width 0.25) (layer "F.Cu") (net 11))
 (segment (start 132.18 89.23) (end 131.95 89.23) (width 0.25) (layer "F.Cu") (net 11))
 (segment (start 129.71 95.39) (end 132.19 97.87) (width 0.25) (layer "F.Cu") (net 11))
 (segment (start 130.271827 101.19) (end 129.81 101.19) (width 0.25) (layer "F.Cu") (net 11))
 (segment (start 132.19 97.87) (end 132.19 99.271827) (width 0.25) (layer "F.Cu") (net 11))
 (segment (start 131.95 89.23) (end 131.95 91.77) (width 0.25) (layer "F.Cu") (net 11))
 (segment (start 133.86 88.13) (end 133.28 88.13) (width 0.25) (layer "F.Cu") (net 11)))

